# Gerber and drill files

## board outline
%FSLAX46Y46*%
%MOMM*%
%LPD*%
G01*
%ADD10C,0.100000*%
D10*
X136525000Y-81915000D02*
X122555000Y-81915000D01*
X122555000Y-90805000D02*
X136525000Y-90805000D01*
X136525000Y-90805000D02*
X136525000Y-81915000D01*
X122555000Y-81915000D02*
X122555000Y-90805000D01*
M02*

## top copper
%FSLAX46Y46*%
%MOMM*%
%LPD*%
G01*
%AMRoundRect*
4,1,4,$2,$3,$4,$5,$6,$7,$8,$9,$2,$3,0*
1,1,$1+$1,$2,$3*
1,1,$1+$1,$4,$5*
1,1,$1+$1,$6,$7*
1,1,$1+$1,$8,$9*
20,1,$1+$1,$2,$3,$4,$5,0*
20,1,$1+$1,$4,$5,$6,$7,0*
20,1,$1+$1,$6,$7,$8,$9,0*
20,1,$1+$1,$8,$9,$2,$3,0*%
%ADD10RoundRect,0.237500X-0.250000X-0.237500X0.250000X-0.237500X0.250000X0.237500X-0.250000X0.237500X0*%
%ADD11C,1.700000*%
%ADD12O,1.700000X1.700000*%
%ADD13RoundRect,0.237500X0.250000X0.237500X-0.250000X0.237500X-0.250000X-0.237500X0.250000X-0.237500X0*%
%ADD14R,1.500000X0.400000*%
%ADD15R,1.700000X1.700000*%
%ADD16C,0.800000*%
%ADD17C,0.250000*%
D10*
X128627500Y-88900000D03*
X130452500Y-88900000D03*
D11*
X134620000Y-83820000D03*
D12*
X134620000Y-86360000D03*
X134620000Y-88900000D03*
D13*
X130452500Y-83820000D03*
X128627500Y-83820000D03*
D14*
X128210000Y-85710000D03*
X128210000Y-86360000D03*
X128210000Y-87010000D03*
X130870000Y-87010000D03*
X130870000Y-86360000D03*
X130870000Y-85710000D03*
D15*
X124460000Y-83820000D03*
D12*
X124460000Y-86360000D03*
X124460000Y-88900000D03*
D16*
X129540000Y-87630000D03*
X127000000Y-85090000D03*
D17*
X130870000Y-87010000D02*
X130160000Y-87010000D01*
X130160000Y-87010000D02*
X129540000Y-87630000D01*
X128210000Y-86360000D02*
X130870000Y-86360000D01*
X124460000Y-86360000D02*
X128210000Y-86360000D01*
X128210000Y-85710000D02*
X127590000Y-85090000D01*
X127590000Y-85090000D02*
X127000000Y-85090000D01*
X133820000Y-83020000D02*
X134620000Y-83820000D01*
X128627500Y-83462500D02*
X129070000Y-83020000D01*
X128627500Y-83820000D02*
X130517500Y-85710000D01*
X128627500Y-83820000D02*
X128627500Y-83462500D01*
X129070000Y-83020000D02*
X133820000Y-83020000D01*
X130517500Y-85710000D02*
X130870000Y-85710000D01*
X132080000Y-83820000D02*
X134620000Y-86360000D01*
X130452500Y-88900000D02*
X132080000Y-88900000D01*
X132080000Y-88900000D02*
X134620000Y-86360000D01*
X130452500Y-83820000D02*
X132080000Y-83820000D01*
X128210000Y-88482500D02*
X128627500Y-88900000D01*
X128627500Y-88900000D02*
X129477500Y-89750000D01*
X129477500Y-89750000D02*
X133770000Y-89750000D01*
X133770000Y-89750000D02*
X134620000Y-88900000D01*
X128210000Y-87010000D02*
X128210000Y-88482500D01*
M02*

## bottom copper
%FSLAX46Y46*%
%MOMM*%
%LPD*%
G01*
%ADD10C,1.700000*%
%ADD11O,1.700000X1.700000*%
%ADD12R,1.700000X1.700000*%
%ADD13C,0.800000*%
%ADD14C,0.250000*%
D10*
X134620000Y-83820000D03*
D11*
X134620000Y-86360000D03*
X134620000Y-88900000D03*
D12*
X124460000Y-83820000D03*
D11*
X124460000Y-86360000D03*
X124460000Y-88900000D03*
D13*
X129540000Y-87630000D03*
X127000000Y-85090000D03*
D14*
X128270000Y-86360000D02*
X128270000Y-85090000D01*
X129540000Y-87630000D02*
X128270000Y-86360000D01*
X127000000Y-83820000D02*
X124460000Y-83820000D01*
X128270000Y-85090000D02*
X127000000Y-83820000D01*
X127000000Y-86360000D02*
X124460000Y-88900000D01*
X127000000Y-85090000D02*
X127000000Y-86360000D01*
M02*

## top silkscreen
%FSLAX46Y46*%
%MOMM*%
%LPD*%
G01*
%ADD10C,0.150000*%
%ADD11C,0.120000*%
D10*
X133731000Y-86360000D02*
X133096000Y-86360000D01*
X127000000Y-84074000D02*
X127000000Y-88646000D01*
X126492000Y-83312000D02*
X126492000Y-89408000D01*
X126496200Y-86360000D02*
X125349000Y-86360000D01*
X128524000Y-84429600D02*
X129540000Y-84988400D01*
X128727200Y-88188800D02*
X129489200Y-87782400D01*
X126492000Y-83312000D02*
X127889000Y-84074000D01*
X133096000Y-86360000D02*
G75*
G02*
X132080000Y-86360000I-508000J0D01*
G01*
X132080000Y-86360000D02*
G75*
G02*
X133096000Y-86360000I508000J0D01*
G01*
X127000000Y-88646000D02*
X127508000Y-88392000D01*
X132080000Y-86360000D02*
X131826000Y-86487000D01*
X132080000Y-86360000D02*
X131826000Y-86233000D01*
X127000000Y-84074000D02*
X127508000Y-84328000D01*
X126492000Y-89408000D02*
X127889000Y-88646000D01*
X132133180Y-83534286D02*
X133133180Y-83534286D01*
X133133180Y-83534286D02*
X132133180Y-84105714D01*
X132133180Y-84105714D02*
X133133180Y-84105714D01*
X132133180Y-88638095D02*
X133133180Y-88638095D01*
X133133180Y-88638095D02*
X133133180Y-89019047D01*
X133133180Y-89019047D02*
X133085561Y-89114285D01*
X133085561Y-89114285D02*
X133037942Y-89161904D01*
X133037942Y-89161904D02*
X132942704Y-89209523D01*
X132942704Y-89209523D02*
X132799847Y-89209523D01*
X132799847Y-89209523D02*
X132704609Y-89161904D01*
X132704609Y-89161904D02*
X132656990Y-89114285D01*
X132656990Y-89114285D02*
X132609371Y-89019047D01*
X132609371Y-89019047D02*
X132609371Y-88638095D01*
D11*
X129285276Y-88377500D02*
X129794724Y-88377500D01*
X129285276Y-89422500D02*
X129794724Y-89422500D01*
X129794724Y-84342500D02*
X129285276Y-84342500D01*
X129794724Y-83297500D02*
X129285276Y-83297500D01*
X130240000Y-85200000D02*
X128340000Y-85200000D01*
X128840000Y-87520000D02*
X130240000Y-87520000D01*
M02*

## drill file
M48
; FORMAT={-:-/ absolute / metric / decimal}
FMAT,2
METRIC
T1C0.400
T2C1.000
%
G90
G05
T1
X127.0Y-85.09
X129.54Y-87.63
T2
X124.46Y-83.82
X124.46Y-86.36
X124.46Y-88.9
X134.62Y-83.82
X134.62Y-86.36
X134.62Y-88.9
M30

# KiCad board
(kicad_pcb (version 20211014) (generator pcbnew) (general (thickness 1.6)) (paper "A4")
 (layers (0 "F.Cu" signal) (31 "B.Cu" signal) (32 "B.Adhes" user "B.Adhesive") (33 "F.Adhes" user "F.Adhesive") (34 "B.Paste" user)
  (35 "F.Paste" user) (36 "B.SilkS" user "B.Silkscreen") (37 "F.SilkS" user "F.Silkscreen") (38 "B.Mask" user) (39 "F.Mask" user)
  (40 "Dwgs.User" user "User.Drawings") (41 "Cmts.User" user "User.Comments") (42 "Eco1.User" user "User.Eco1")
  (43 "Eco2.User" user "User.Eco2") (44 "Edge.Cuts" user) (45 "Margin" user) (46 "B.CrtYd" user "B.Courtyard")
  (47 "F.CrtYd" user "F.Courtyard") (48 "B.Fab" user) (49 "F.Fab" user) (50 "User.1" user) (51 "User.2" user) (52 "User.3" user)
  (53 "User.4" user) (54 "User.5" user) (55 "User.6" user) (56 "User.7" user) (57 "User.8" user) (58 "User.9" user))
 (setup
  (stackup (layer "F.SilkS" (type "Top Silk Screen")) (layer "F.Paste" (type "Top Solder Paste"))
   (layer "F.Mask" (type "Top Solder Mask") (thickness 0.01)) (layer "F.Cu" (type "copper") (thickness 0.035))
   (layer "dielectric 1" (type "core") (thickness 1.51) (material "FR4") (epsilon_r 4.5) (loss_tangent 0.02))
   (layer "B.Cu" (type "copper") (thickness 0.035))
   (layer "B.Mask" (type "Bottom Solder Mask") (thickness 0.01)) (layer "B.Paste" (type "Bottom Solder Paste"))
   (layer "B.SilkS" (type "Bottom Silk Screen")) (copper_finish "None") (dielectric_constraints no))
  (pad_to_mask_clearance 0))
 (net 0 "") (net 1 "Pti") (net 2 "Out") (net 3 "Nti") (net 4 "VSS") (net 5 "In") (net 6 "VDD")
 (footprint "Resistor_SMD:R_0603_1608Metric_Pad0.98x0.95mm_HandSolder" (layer "F.Cu") (at 129.54 88.9)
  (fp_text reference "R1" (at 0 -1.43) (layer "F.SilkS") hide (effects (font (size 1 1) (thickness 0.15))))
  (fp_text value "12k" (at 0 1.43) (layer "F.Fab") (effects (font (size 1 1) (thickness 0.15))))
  (fp_line (start -0.254724 -0.5225) (end 0.254724 -0.5225) (layer "F.SilkS") (width 0.12))
  (fp_line (start -0.254724 0.5225) (end 0.254724 0.5225) (layer "F.SilkS") (width 0.12))
  (pad "1" smd roundrect (at -0.9125 0) (size 0.975 0.95) (layers "F.Cu" "F.Paste" "F.Mask") (roundrect_rratio 0.25) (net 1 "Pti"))
  (pad "2" smd roundrect (at 0.9125 0) (size 0.975 0.95) (layers "F.Cu" "F.Paste" "F.Mask") (roundrect_rratio 0.25) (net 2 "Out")))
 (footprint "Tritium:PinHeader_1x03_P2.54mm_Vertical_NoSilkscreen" (layer "F.Cu") (at 134.62 83.82)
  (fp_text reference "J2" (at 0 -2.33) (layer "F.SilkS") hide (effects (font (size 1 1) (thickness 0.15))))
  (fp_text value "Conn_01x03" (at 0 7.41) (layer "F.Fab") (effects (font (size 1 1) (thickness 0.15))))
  (pad "1" thru_hole circle (at 0 0) (size 1.7 1.7) (drill 1) (layers *.Cu *.Mask) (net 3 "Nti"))
  (pad "2" thru_hole oval (at 0 2.54) (size 1.7 1.7) (drill 1) (layers *.Cu *.Mask) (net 2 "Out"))
  (pad "3" thru_hole oval (at 0 5.08) (size 1.7 1.7) (drill 1) (layers *.Cu *.Mask) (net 1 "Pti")))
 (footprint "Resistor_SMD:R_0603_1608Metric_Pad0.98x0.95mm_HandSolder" (layer "F.Cu") (at 129.54 83.82 180)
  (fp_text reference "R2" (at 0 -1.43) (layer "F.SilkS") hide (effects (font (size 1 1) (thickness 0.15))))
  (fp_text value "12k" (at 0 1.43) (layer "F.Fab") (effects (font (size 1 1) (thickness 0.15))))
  (fp_line (start -0.254724 -0.5225) (end 0.254724 -0.5225) (layer "F.SilkS") (width 0.12))
  (fp_line (start -0.254724 0.5225) (end 0.254724 0.5225) (layer "F.SilkS") (width 0.12))
  (pad "1" smd roundrect (at -0.9125 0 180) (size 0.975 0.95) (layers "F.Cu" "F.Paste" "F.Mask") (roundrect_rratio 0.25) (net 2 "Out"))
  (pad "2" smd roundrect (at 0.9125 0 180) (size 0.975 0.95) (layers "F.Cu" "F.Paste" "F.Mask") (roundrect_rratio 0.25) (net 3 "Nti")))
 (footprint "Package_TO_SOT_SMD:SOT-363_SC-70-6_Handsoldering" (layer "F.Cu") (at 129.54 86.36)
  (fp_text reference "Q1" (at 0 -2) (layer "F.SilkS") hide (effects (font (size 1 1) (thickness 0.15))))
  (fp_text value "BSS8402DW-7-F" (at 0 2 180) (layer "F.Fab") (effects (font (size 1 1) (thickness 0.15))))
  (fp_line (start 0.7 -1.16) (end -1.2 -1.16) (layer "F.SilkS") (width 0.12))
  (fp_line (start -0.7 1.16) (end 0.7 1.16) (layer "F.SilkS") (width 0.12))
  (pad "1" smd rect (at -1.33 -0.65) (size 1.5 0.4) (layers "F.Cu" "F.Paste" "F.Mask") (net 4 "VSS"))
  (pad "2" smd rect (at -1.33 0) (size 1.5 0.4) (layers "F.Cu" "F.Paste" "F.Mask") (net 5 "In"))
  (pad "3" smd rect (at -1.33 0.65) (size 1.5 0.4) (layers "F.Cu" "F.Paste" "F.Mask") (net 1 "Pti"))
  (pad "4" smd rect (at 1.33 0.65) (size 1.5 0.4) (layers "F.Cu" "F.Paste" "F.Mask") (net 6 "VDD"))
  (pad "5" smd rect (at 1.33 0) (size 1.5 0.4) (layers "F.Cu" "F.Paste" "F.Mask") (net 5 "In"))
  (pad "6" smd rect (at 1.33 -0.65) (size 1.5 0.4) (layers "F.Cu" "F.Paste" "F.Mask") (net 3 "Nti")))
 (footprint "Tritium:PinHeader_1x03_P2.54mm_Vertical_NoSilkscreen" (layer "F.Cu") (at 124.46 83.82)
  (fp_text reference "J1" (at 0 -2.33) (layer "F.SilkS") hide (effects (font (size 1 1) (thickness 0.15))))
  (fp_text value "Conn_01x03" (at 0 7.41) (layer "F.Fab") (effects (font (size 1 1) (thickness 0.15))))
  (pad "1" thru_hole rect (at 0 0) (size 1.7 1.7) (drill 1) (layers *.Cu *.Mask) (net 6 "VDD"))
  (pad "2" thru_hole oval (at 0 2.54) (size 1.7 1.7) (drill 1) (layers *.Cu *.Mask) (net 5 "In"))
  (pad "3" thru_hole oval (at 0 5.08) (size 1.7 1.7) (drill 1) (layers *.Cu *.Mask) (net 4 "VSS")))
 (gr_line (start 133.731 86.36) (end 133.096 86.36) (layer "F.SilkS") (width 0.15))
 (gr_line (start 127 84.074) (end 127 88.646) (layer "F.SilkS") (width 0.15))
 (gr_line (start 126.492 83.312) (end 126.492 89.408) (layer "F.SilkS") (width 0.15))
 (gr_line (start 126.4962 86.36) (end 125.349 86.36) (layer "F.SilkS") (width 0.15))
 (gr_line (start 128.524 84.4296) (end 129.54 84.9884) (layer "F.SilkS") (width 0.15))
 (gr_line (start 128.7272 88.1888) (end 129.4892 87.7824) (layer "F.SilkS") (width 0.15))
 (gr_line (start 126.492 83.312) (end 127.889 84.074) (layer "F.SilkS") (width 0.15))
 (gr_circle (center 132.588 86.36) (end 132.08 86.36) (layer "F.SilkS") (width 0.15) (fill none))
 (gr_line (start 127 88.646) (end 127.508 88.392) (layer "F.SilkS") (width 0.15))
 (gr_line (start 132.08 86.36) (end 131.826 86.487) (layer "F.SilkS") (width 0.15))
 (gr_line (start 132.08 86.36) (end 131.826 86.233) (layer "F.SilkS") (width 0.15))
 (gr_line (start 127 84.074) (end 127.508 84.328) (layer "F.SilkS") (width 0.15))
 (gr_line (start 126.492 89.408) (end 127.889 88.646) (layer "F.SilkS") (width 0.15))
 (gr_line (start 136.525 81.915) (end 122.555 81.915) (layer "Edge.Cuts") (width 0.1))
 (gr_line (start 122.555 90.805) (end 136.525 90.805) (layer "Edge.Cuts") (width 0.1))
 (gr_line (start 136.525 90.805) (end 136.525 81.915) (layer "Edge.Cuts") (width 0.1))
 (gr_line (start 122.555 81.915) (end 122.555 90.805) (layer "Edge.Cuts") (width 0.1))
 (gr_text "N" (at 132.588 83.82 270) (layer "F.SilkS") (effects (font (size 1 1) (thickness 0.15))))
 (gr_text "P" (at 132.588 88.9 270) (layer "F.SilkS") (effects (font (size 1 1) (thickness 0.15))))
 (segment (start 130.87 87.01) (end 130.16 87.01) (width 0.25) (layer "F.Cu") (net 6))
 (segment (start 130.16 87.01) (end 129.54 87.63) (width 0.25) (layer "F.Cu") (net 6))
 (via (at 129.54 87.63) (size 0.8) (drill 0.4) (layers "F.Cu" "B.Cu") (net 6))
 (segment (start 128.27 86.36) (end 128.27 85.09) (width 0.25) (layer "B.Cu") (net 6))
 (segment (start 129.54 87.63) (end 128.27 86.36) (width 0.25) (layer "B.Cu") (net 6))
 (segment (start 127 83.82) (end 124.46 83.82) (width 0.25) (layer "B.Cu") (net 6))
 (segment (start 128.27 85.09) (end 127 83.82) (width 0.25) (layer "B.Cu") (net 6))
 (segment (start 128.21 86.36) (end 130.87 86.36) (width 0.25) (layer "F.Cu") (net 5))
 (segment (start 124.46 86.36) (end 128.21 86.36) (width 0.25) (layer "F.Cu") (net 5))
 (segment (start 128.21 85.71) (end 127.59 85.09) (width 0.25) (layer "F.Cu") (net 4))
 (segment (start 127.59 85.09) (end 127 85.09) (width 0.25) (layer "F.Cu") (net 4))
 (via (at 127 85.09) (size 0.8) (drill 0.4) (layers "F.Cu" "B.Cu") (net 4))
 (segment (start 127 86.36) (end 124.46 88.9) (width 0.25) (layer "B.Cu") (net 4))
 (segment (start 127 85.09) (end 127 86.36) (width 0.25) (layer "B.Cu") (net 4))
 (segment (start 133.82 83.02) (end 134.62 83.82) (width 0.25) (layer "F.Cu") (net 3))
 (segment (start 128.6275 83.4625) (end 129.07 83.02) (width 0.25) (layer "F.Cu") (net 3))
 (segment (start 128.6275 83.82) (end 130.5175 85.71) (width 0.25) (layer "F.Cu") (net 3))
 (segment (start 128.6275 83.82) (end 128.6275 83.4625) (width 0.25) (layer "F.Cu") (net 3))
 (segment (start 129.07 83.02) (end 133.82 83.02) (width 0.25) (layer "F.Cu") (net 3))
 (segment (start 130.5175 85.71) (end 130.87 85.71) (width 0.25) (layer "F.Cu") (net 3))
 (segment (start 132.08 83.82) (end 134.62 86.36) (width 0.25) (layer "F.Cu") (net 2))
 (segment (start 130.4525 88.9) (end 132.08 88.9) (width 0.25) (layer "F.Cu") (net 2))
 (segment (start 132.08 88.9) (end 134.62 86.36) (width 0.25) (layer "F.Cu") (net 2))
 (segment (start 130.4525 83.82) (end 132.08 83.82) (width 0.25) (layer "F.Cu") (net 2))
 (segment (start 128.21 88.4825) (end 128.6275 88.9) (width 0.25) (layer "F.Cu") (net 1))
 (segment (start 128.6275 88.9) (end 129.4775 89.75) (width 0.25) (layer "F.Cu") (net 1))
 (segment (start 129.4775 89.75) (end 133.77 89.75) (width 0.25) (layer "F.Cu") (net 1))
 (segment (start 133.77 89.75) (end 134.62 88.9) (width 0.25) (layer "F.Cu") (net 1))
 (segment (start 128.21 87.01) (end 128.21 88.4825) (width 0.25) (layer "F.Cu") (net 1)))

